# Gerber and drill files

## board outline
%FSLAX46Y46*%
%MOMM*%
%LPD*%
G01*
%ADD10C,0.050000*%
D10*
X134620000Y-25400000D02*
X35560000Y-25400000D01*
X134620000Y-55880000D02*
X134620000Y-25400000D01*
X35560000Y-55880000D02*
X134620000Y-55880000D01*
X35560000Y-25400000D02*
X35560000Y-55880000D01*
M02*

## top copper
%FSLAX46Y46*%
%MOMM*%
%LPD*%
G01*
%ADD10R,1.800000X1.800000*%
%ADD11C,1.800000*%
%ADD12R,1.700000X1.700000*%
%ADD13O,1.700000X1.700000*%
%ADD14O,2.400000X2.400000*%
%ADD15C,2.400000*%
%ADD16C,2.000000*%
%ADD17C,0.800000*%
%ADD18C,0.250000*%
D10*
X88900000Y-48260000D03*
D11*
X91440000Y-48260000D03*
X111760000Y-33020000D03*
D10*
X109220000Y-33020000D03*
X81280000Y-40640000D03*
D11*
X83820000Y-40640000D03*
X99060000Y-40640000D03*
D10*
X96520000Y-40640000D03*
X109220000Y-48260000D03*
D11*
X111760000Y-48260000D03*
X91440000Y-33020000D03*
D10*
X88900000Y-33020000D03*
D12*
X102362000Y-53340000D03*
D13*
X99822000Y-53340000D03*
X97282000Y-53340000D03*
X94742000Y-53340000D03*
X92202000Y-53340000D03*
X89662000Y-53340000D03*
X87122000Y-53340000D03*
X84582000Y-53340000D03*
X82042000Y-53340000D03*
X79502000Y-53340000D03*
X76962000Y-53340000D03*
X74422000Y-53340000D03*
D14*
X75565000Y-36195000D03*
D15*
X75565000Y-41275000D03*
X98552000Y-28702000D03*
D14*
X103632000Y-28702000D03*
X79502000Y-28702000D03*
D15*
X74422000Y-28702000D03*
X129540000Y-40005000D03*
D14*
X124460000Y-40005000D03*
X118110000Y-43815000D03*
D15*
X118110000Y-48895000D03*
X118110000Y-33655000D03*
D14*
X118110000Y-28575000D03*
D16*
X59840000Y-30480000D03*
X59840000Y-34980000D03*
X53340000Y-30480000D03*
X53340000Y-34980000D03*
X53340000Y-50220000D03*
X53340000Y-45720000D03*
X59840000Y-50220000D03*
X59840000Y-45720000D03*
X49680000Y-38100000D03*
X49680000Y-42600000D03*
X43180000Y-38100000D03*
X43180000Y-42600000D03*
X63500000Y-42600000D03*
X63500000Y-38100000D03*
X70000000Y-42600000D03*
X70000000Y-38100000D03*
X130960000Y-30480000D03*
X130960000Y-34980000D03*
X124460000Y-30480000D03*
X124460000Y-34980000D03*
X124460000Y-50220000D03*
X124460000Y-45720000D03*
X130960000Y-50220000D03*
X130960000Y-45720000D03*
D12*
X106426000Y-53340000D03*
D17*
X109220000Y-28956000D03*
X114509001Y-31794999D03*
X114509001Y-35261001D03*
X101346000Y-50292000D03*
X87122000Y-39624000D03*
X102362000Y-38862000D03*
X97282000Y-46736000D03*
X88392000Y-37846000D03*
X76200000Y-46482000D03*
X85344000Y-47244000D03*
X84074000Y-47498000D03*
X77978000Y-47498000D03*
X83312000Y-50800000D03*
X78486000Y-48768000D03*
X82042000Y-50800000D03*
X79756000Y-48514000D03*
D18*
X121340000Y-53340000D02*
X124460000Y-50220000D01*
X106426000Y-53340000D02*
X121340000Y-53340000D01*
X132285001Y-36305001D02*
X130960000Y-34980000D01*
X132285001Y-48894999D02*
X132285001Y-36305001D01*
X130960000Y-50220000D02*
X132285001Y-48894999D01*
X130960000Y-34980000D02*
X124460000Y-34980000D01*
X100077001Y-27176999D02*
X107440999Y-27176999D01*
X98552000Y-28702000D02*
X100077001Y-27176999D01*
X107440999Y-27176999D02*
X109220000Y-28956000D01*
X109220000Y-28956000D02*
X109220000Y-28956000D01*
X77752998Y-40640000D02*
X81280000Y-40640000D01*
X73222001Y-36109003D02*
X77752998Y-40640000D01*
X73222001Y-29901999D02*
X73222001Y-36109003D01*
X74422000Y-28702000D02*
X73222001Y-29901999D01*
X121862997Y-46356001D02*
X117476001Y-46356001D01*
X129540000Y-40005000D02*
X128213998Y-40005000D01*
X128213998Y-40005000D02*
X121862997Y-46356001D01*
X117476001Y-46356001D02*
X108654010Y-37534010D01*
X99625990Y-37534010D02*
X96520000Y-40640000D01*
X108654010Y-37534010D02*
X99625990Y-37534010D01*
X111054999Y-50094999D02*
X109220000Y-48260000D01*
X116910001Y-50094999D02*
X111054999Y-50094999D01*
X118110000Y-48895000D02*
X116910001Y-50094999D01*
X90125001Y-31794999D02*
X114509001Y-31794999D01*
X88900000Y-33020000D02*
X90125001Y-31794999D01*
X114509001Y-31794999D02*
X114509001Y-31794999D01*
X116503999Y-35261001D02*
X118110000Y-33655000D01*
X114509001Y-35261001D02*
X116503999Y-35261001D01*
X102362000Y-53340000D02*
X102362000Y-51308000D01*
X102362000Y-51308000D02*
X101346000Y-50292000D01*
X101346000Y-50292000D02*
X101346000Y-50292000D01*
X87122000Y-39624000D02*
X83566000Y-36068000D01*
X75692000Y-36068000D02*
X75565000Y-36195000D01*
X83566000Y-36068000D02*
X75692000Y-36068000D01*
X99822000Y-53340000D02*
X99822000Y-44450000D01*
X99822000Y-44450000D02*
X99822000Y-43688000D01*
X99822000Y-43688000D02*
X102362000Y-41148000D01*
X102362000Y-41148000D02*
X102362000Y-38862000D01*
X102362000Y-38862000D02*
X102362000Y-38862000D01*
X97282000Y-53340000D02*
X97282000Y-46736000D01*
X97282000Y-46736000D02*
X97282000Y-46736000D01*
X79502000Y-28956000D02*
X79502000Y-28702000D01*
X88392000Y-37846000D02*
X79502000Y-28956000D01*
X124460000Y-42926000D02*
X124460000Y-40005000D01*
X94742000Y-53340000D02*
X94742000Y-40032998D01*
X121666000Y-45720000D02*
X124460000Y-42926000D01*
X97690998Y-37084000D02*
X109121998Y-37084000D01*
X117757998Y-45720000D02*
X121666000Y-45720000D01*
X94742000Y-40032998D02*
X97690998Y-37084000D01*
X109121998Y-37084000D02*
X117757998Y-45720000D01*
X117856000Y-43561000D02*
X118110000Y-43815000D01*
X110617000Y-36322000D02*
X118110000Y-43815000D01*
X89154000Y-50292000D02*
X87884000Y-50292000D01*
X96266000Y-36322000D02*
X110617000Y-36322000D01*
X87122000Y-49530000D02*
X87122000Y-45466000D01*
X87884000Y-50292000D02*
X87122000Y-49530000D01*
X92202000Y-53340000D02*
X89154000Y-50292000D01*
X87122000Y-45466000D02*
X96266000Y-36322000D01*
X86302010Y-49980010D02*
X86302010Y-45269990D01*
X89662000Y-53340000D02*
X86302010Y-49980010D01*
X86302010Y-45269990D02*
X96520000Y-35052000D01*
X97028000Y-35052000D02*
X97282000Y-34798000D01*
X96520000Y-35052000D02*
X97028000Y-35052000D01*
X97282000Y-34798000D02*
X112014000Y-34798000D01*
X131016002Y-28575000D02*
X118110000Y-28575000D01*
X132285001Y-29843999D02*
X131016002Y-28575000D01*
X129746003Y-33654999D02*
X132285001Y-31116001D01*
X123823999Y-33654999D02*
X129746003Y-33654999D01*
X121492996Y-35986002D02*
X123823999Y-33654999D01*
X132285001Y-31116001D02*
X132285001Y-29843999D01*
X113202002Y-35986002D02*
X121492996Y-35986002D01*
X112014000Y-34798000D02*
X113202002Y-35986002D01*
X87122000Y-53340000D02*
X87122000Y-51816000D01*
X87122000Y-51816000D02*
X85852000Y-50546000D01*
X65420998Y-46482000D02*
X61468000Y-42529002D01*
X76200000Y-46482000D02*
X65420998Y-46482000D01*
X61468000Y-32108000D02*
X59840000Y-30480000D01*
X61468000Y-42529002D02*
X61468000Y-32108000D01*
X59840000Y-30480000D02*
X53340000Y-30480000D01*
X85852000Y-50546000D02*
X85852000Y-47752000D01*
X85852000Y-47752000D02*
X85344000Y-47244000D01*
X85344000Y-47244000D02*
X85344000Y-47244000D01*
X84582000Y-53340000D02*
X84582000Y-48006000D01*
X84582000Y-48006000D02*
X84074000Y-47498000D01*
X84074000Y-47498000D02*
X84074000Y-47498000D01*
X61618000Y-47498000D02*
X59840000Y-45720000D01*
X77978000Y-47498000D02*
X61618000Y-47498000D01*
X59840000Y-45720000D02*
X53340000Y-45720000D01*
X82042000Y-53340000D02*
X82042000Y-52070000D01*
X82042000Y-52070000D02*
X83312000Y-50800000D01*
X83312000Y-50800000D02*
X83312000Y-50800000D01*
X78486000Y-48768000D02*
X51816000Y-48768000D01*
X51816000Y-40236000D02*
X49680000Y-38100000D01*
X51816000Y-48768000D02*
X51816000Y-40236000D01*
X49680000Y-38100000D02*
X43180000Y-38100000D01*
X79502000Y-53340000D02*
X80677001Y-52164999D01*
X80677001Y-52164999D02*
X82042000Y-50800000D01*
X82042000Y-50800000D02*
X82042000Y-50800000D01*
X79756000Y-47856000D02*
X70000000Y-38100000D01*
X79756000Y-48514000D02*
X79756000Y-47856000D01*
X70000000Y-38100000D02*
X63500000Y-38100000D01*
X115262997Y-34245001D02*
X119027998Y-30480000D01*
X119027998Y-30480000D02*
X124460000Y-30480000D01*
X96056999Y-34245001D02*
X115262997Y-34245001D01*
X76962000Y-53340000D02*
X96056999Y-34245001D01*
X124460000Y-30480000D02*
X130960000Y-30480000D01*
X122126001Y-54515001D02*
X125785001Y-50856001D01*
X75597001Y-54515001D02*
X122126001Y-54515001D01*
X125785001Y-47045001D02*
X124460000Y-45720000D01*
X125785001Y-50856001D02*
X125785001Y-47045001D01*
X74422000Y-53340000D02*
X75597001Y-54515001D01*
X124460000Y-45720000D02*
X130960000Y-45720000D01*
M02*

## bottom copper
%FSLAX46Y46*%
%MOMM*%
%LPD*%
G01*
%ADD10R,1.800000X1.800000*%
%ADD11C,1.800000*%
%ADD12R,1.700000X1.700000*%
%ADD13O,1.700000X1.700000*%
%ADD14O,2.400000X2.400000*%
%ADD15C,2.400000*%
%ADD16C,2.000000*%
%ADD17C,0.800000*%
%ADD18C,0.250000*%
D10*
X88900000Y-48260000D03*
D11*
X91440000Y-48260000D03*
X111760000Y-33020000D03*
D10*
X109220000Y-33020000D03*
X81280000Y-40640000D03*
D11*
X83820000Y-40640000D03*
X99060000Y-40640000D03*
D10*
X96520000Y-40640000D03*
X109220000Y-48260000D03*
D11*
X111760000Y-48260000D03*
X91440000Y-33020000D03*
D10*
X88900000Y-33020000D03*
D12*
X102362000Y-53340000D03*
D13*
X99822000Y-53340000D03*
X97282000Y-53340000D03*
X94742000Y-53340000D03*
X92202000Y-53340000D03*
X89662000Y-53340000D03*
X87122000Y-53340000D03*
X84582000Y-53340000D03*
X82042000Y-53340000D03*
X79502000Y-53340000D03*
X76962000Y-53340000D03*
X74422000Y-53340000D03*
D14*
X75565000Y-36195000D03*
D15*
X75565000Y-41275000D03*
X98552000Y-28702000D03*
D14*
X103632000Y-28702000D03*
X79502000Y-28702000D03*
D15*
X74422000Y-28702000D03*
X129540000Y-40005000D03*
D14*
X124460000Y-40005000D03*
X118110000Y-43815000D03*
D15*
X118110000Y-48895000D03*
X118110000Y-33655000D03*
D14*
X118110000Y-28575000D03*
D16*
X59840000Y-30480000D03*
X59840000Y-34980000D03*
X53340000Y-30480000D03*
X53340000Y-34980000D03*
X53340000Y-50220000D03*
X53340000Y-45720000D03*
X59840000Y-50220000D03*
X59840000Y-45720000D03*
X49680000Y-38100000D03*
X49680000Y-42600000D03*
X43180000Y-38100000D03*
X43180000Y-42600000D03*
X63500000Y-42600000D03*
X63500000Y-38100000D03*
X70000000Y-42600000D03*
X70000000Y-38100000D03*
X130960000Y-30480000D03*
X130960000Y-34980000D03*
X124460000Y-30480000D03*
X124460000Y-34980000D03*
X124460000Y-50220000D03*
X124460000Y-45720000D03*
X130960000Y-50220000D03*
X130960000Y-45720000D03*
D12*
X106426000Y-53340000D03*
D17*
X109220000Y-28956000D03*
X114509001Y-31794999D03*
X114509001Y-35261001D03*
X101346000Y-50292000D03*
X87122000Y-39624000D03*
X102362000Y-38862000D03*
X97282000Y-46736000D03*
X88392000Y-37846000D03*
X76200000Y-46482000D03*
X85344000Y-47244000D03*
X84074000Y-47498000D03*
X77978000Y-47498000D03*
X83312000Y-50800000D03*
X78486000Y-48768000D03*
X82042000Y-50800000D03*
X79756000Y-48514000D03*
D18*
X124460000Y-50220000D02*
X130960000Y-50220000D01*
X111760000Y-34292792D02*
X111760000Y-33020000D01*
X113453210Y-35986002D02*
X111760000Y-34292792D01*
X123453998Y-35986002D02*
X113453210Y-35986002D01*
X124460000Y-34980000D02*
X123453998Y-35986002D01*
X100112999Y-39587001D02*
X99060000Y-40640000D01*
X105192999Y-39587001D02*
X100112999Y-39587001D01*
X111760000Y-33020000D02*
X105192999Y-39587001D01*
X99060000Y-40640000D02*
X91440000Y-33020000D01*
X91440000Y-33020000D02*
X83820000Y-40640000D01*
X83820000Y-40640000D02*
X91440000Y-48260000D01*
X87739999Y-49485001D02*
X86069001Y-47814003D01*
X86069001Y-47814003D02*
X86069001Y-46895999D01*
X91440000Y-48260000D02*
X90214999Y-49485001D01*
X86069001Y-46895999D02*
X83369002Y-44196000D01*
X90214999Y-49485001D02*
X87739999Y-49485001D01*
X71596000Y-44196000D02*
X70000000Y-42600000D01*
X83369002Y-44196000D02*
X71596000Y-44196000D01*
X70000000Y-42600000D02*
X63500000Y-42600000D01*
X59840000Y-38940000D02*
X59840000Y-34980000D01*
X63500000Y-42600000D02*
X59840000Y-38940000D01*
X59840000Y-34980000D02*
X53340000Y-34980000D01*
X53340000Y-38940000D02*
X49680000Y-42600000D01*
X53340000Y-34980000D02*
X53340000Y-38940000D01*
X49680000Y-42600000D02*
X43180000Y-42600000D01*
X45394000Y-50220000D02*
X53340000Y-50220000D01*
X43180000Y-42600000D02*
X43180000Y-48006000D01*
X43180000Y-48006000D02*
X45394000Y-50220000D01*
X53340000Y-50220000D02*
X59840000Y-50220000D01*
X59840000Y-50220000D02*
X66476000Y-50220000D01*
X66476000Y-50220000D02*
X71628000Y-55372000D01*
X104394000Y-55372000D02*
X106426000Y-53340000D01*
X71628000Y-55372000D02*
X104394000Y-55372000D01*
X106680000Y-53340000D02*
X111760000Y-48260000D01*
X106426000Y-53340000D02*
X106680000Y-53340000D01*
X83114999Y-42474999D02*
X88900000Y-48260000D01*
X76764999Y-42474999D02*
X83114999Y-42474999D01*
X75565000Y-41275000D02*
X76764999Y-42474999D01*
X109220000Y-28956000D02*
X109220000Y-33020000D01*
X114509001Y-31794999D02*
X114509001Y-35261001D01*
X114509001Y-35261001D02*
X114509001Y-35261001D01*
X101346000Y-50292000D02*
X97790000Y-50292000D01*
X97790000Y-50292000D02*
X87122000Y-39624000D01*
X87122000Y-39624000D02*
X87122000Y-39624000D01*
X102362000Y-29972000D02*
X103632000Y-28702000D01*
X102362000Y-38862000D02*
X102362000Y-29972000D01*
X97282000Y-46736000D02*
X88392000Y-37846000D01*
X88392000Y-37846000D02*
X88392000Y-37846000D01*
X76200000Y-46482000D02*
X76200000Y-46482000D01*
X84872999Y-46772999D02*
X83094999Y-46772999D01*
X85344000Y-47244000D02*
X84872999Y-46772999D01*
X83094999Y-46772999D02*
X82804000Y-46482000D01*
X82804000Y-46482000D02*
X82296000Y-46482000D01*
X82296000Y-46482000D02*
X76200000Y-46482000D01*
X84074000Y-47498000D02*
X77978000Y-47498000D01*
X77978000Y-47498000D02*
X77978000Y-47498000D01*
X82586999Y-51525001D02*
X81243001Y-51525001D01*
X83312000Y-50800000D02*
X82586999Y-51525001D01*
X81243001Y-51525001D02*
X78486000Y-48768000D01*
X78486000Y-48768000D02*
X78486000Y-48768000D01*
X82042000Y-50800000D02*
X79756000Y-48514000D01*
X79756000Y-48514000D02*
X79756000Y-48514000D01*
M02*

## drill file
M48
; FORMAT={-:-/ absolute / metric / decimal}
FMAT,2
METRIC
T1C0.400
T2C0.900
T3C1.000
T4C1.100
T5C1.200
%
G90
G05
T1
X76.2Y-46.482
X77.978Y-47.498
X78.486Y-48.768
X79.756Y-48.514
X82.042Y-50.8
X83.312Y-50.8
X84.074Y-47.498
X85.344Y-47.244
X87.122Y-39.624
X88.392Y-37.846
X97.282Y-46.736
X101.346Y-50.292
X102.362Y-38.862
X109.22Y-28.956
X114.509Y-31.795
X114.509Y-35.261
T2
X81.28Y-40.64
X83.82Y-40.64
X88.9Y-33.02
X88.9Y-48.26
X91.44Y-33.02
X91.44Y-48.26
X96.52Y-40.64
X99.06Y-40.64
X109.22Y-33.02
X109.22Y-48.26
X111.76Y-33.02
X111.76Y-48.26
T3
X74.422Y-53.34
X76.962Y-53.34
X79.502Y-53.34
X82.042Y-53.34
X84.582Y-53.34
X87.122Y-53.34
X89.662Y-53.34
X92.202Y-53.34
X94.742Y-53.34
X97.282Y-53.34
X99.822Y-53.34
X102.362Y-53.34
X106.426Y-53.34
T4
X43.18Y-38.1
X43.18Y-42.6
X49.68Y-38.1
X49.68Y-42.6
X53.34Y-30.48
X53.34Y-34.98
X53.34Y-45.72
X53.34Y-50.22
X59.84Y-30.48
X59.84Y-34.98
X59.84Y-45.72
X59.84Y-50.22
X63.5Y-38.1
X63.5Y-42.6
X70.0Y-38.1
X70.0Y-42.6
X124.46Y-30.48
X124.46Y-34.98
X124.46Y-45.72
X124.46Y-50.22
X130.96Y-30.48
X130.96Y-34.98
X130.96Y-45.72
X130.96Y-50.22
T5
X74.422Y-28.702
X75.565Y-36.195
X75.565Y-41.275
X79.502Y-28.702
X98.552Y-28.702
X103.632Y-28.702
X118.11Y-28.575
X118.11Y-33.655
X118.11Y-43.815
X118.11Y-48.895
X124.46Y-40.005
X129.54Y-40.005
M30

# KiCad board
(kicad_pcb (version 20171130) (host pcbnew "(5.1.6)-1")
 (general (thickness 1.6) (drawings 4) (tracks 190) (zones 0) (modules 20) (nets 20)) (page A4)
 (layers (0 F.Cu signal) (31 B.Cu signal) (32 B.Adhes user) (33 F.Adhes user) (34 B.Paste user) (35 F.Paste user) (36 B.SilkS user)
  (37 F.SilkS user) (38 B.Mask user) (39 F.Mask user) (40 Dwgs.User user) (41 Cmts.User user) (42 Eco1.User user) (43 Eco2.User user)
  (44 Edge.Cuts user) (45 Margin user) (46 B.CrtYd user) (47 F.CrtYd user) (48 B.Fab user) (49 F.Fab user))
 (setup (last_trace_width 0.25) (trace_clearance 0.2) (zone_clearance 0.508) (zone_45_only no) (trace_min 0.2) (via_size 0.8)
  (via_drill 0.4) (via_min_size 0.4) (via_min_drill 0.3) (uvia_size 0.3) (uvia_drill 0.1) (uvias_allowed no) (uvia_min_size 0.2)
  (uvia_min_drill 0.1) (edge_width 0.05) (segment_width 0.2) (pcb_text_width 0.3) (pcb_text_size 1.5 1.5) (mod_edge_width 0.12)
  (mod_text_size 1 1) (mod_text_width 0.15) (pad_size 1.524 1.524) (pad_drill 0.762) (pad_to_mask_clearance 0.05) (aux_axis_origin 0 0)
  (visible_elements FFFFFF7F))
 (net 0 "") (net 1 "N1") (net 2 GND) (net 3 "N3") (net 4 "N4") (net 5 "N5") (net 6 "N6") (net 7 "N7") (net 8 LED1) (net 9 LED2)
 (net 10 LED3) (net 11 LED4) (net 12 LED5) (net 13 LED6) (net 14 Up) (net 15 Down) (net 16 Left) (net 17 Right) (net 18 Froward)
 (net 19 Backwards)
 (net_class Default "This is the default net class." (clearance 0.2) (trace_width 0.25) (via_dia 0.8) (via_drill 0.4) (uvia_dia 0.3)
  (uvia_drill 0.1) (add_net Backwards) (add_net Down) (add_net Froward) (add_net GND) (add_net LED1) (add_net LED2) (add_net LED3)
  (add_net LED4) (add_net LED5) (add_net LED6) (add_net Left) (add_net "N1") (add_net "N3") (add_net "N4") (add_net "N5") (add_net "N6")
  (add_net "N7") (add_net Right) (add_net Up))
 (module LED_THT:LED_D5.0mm (layer F.Cu) (at 88.9 48.26)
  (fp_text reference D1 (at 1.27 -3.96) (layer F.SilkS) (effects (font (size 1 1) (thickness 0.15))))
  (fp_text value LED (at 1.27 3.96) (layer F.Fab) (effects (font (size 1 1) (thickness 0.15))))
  (pad 1 thru_hole rect (at 0 0) (size 1.8 1.8) (drill 0.9) (layers *.Cu *.Mask) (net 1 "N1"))
  (pad 2 thru_hole circle (at 2.54 0) (size 1.8 1.8) (drill 0.9) (layers *.Cu *.Mask) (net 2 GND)))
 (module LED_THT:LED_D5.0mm (layer F.Cu) (at 109.22 33.02)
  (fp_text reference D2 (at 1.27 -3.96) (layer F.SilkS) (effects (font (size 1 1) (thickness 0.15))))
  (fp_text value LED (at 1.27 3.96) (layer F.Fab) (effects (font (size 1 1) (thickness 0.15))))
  (pad 2 thru_hole circle (at 2.54 0) (size 1.8 1.8) (drill 0.9) (layers *.Cu *.Mask) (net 2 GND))
  (pad 1 thru_hole rect (at 0 0) (size 1.8 1.8) (drill 0.9) (layers *.Cu *.Mask) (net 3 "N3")))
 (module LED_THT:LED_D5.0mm (layer F.Cu) (at 81.28 40.64)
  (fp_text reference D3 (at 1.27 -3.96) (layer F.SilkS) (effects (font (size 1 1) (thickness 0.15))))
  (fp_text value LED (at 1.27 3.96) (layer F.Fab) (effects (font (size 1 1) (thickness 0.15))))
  (pad 1 thru_hole rect (at 0 0) (size 1.8 1.8) (drill 0.9) (layers *.Cu *.Mask) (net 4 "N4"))
  (pad 2 thru_hole circle (at 2.54 0) (size 1.8 1.8) (drill 0.9) (layers *.Cu *.Mask) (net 2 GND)))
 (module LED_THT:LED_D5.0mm (layer F.Cu) (at 96.52 40.64)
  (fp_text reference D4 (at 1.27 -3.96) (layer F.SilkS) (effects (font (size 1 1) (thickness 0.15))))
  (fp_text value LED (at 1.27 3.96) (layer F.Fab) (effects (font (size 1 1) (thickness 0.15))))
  (pad 2 thru_hole circle (at 2.54 0) (size 1.8 1.8) (drill 0.9) (layers *.Cu *.Mask) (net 2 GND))
  (pad 1 thru_hole rect (at 0 0) (size 1.8 1.8) (drill 0.9) (layers *.Cu *.Mask) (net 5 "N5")))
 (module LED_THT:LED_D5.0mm (layer F.Cu) (at 109.22 48.26)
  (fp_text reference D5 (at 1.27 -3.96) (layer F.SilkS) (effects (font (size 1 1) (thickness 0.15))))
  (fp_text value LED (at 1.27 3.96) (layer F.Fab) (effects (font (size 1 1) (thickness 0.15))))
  (pad 1 thru_hole rect (at 0 0) (size 1.8 1.8) (drill 0.9) (layers *.Cu *.Mask) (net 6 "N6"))
  (pad 2 thru_hole circle (at 2.54 0) (size 1.8 1.8) (drill 0.9) (layers *.Cu *.Mask) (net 2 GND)))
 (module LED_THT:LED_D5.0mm (layer F.Cu) (at 88.9 33.02)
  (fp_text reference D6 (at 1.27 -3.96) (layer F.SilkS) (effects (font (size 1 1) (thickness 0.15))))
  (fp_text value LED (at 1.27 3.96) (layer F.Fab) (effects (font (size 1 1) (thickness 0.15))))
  (pad 2 thru_hole circle (at 2.54 0) (size 1.8 1.8) (drill 0.9) (layers *.Cu *.Mask) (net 2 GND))
  (pad 1 thru_hole rect (at 0 0) (size 1.8 1.8) (drill 0.9) (layers *.Cu *.Mask) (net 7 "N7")))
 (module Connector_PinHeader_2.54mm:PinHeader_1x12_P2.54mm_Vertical (layer F.Cu) (at 102.362 53.34 270)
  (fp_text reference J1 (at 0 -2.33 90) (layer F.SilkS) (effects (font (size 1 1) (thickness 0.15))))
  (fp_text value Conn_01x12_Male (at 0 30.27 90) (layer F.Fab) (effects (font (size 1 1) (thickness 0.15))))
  (pad 1 thru_hole rect (at 0 0 270) (size 1.7 1.7) (drill 1) (layers *.Cu *.Mask) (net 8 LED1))
  (pad 2 thru_hole oval (at 0 2.54 270) (size 1.7 1.7) (drill 1) (layers *.Cu *.Mask) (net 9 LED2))
  (pad 3 thru_hole oval (at 0 5.08 270) (size 1.7 1.7) (drill 1) (layers *.Cu *.Mask) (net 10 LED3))
  (pad 4 thru_hole oval (at 0 7.62 270) (size 1.7 1.7) (drill 1) (layers *.Cu *.Mask) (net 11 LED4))
  (pad 5 thru_hole oval (at 0 10.16 270) (size 1.7 1.7) (drill 1) (layers *.Cu *.Mask) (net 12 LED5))
  (pad 6 thru_hole oval (at 0 12.7 270) (size 1.7 1.7) (drill 1) (layers *.Cu *.Mask) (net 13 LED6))
  (pad 7 thru_hole oval (at 0 15.24 270) (size 1.7 1.7) (drill 1) (layers *.Cu *.Mask) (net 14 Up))
  (pad 8 thru_hole oval (at 0 17.78 270) (size 1.7 1.7) (drill 1) (layers *.Cu *.Mask) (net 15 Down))
  (pad 9 thru_hole oval (at 0 20.32 270) (size 1.7 1.7) (drill 1) (layers *.Cu *.Mask) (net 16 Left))
  (pad 10 thru_hole oval (at 0 22.86 270) (size 1.7 1.7) (drill 1) (layers *.Cu *.Mask) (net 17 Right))
  (pad 11 thru_hole oval (at 0 25.4 270) (size 1.7 1.7) (drill 1) (layers *.Cu *.Mask) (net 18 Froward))
  (pad 12 thru_hole oval (at 0 27.94 270) (size 1.7 1.7) (drill 1) (layers *.Cu *.Mask) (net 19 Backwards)))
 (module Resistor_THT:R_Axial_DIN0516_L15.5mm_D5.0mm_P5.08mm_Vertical (layer F.Cu) (at 75.565 41.275 90)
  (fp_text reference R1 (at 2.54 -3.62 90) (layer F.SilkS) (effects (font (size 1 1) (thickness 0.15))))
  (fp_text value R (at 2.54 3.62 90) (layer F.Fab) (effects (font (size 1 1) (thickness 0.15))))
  (pad 2 thru_hole oval (at 5.08 0 90) (size 2.4 2.4) (drill 1.2) (layers *.Cu *.Mask) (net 8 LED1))
  (pad 1 thru_hole circle (at 0 0 90) (size 2.4 2.4) (drill 1.2) (layers *.Cu *.Mask) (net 1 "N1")))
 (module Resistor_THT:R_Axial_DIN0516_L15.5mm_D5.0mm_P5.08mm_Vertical (layer F.Cu) (at 98.552 28.702)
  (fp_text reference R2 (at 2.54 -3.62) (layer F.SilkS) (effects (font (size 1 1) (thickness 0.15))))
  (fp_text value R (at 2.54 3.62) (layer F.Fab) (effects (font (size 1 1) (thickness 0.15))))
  (pad 1 thru_hole circle (at 0 0) (size 2.4 2.4) (drill 1.2) (layers *.Cu *.Mask) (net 3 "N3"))
  (pad 2 thru_hole oval (at 5.08 0) (size 2.4 2.4) (drill 1.2) (layers *.Cu *.Mask) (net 9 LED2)))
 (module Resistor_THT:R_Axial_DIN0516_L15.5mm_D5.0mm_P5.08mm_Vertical (layer F.Cu) (at 74.422 28.702)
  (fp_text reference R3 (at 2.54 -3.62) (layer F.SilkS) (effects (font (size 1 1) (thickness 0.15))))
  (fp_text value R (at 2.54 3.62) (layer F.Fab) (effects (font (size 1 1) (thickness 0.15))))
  (pad 2 thru_hole oval (at 5.08 0) (size 2.4 2.4) (drill 1.2) (layers *.Cu *.Mask) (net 10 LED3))
  (pad 1 thru_hole circle (at 0 0) (size 2.4 2.4) (drill 1.2) (layers *.Cu *.Mask) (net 4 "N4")))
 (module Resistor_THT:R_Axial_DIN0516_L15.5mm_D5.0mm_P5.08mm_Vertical (layer F.Cu) (at 129.54 40.005 180)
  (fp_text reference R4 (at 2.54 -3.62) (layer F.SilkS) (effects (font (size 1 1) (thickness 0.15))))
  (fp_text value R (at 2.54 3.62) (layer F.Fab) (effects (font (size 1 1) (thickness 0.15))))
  (pad 1 thru_hole circle (at 0 0 180) (size 2.4 2.4) (drill 1.2) (layers *.Cu *.Mask) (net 5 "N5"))
  (pad 2 thru_hole oval (at 5.08 0 180) (size 2.4 2.4) (drill 1.2) (layers *.Cu *.Mask) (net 11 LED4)))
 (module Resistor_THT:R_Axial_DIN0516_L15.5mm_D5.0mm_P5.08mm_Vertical (layer F.Cu) (at 118.11 48.895 90)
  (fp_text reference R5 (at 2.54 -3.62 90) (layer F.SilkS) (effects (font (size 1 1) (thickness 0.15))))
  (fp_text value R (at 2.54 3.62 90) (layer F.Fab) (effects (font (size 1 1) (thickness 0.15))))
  (pad 2 thru_hole oval (at 5.08 0 90) (size 2.4 2.4) (drill 1.2) (layers *.Cu *.Mask) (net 12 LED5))
  (pad 1 thru_hole circle (at 0 0 90) (size 2.4 2.4) (drill 1.2) (layers *.Cu *.Mask) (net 6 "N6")))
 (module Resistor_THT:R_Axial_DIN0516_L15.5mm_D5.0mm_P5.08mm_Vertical (layer F.Cu) (at 118.11 33.655 90)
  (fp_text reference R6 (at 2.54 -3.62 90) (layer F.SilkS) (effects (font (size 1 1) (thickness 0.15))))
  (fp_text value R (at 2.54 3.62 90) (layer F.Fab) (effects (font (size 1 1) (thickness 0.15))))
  (pad 1 thru_hole circle (at 0 0 90) (size 2.4 2.4) (drill 1.2) (layers *.Cu *.Mask) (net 7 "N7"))
  (pad 2 thru_hole oval (at 5.08 0 90) (size 2.4 2.4) (drill 1.2) (layers *.Cu *.Mask) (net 13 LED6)))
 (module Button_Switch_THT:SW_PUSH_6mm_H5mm (layer F.Cu) (at 53.34 30.48)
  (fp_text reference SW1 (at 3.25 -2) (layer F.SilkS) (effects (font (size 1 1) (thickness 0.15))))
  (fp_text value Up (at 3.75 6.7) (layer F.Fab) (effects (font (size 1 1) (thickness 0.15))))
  (pad 1 thru_hole circle (at 6.5 0 90) (size 2 2) (drill 1.1) (layers *.Cu *.Mask) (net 14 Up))
  (pad 2 thru_hole circle (at 6.5 4.5 90) (size 2 2) (drill 1.1) (layers *.Cu *.Mask) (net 2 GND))
  (pad 1 thru_hole circle (at 0 0 90) (size 2 2) (drill 1.1) (layers *.Cu *.Mask) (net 14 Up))
  (pad 2 thru_hole circle (at 0 4.5 90) (size 2 2) (drill 1.1) (layers *.Cu *.Mask) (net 2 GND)))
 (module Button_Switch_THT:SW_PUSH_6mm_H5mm (layer F.Cu) (at 53.34 45.72)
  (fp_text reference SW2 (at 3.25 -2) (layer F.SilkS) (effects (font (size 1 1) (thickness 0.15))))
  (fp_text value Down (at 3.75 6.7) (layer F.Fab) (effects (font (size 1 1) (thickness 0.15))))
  (pad 2 thru_hole circle (at 0 4.5 90) (size 2 2) (drill 1.1) (layers *.Cu *.Mask) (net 2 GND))
  (pad 1 thru_hole circle (at 0 0 90) (size 2 2) (drill 1.1) (layers *.Cu *.Mask) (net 15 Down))
  (pad 2 thru_hole circle (at 6.5 4.5 90) (size 2 2) (drill 1.1) (layers *.Cu *.Mask) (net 2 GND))
  (pad 1 thru_hole circle (at 6.5 0 90) (size 2 2) (drill 1.1) (layers *.Cu *.Mask) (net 15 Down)))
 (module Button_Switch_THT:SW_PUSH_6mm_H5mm (layer F.Cu) (at 43.18 38.1)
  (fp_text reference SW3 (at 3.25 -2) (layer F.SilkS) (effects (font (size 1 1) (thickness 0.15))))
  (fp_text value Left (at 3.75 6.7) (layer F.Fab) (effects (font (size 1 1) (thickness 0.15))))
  (pad 1 thru_hole circle (at 6.5 0 90) (size 2 2) (drill 1.1) (layers *.Cu *.Mask) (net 16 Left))
  (pad 2 thru_hole circle (at 6.5 4.5 90) (size 2 2) (drill 1.1) (layers *.Cu *.Mask) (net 2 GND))
  (pad 1 thru_hole circle (at 0 0 90) (size 2 2) (drill 1.1) (layers *.Cu *.Mask) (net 16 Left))
  (pad 2 thru_hole circle (at 0 4.5 90) (size 2 2) (drill 1.1) (layers *.Cu *.Mask) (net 2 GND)))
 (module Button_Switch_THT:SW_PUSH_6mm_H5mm (layer F.Cu) (at 63.5 38.1)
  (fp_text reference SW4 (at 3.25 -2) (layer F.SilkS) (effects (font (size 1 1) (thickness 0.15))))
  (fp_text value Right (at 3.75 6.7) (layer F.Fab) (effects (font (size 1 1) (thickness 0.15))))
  (pad 2 thru_hole circle (at 0 4.5 90) (size 2 2) (drill 1.1) (layers *.Cu *.Mask) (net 2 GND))
  (pad 1 thru_hole circle (at 0 0 90) (size 2 2) (drill 1.1) (layers *.Cu *.Mask) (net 17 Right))
  (pad 2 thru_hole circle (at 6.5 4.5 90) (size 2 2) (drill 1.1) (layers *.Cu *.Mask) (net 2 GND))
  (pad 1 thru_hole circle (at 6.5 0 90) (size 2 2) (drill 1.1) (layers *.Cu *.Mask) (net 17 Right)))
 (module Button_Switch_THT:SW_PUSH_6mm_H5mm (layer F.Cu) (at 124.46 30.48)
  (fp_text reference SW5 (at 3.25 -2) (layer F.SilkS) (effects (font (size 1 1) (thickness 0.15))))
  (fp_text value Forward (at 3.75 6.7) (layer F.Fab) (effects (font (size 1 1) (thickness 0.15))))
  (pad 1 thru_hole circle (at 6.5 0 90) (size 2 2) (drill 1.1) (layers *.Cu *.Mask) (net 18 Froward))
  (pad 2 thru_hole circle (at 6.5 4.5 90) (size 2 2) (drill 1.1) (layers *.Cu *.Mask) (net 2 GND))
  (pad 1 thru_hole circle (at 0 0 90) (size 2 2) (drill 1.1) (layers *.Cu *.Mask) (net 18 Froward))
  (pad 2 thru_hole circle (at 0 4.5 90) (size 2 2) (drill 1.1) (layers *.Cu *.Mask) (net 2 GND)))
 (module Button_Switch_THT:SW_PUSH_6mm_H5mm (layer F.Cu) (at 124.46 45.72)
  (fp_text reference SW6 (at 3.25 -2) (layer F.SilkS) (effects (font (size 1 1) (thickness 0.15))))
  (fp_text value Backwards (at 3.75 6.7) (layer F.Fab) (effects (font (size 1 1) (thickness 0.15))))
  (pad 2 thru_hole circle (at 0 4.5 90) (size 2 2) (drill 1.1) (layers *.Cu *.Mask) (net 2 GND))
  (pad 1 thru_hole circle (at 0 0 90) (size 2 2) (drill 1.1) (layers *.Cu *.Mask) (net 19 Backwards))
  (pad 2 thru_hole circle (at 6.5 4.5 90) (size 2 2) (drill 1.1) (layers *.Cu *.Mask) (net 2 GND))
  (pad 1 thru_hole circle (at 6.5 0 90) (size 2 2) (drill 1.1) (layers *.Cu *.Mask) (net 19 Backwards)))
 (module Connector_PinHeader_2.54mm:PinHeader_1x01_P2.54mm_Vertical (layer F.Cu) (at 106.426 53.34)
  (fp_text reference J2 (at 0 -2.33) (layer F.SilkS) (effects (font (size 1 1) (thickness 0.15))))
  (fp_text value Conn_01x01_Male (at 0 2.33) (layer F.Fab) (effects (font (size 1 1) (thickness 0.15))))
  (pad 1 thru_hole rect (at 0 0) (size 1.7 1.7) (drill 1) (layers *.Cu *.Mask) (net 2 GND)))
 (gr_line (start 134.62 25.4) (end 35.56 25.4) (layer Edge.Cuts) (width 0.05))
 (gr_line (start 134.62 55.88) (end 134.62 25.4) (layer Edge.Cuts) (width 0.05))
 (gr_line (start 35.56 55.88) (end 134.62 55.88) (layer Edge.Cuts) (width 0.05))
 (gr_line (start 35.56 25.4) (end 35.56 55.88) (layer Edge.Cuts) (width 0.05))
 (segment (start 121.34 53.34) (end 124.46 50.22) (width 0.25) (layer F.Cu) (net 2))
 (segment (start 106.426 53.34) (end 121.34 53.34) (width 0.25) (layer F.Cu) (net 2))
 (segment (start 124.46 50.22) (end 130.96 50.22) (width 0.25) (layer B.Cu) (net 2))
 (segment (start 132.285001 36.305001) (end 130.96 34.98) (width 0.25) (layer F.Cu) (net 2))
 (segment (start 132.285001 48.894999) (end 132.285001 36.305001) (width 0.25) (layer F.Cu) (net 2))
 (segment (start 130.96 50.22) (end 132.285001 48.894999) (width 0.25) (layer F.Cu) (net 2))
 (segment (start 130.96 34.98) (end 124.46 34.98) (width 0.25) (layer F.Cu) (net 2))
 (segment (start 111.76 34.292792) (end 111.76 33.02) (width 0.25) (layer B.Cu) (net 2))
 (segment (start 113.45321 35.986002) (end 111.76 34.292792) (width 0.25) (layer B.Cu) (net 2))
 (segment (start 123.453998 35.986002) (end 113.45321 35.986002) (width 0.25) (layer B.Cu) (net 2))
 (segment (start 124.46 34.98) (end 123.453998 35.986002) (width 0.25) (layer B.Cu) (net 2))
 (segment (start 100.112999 39.587001) (end 99.06 40.64) (width 0.25) (layer B.Cu) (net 2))
 (segment (start 105.192999 39.587001) (end 100.112999 39.587001) (width 0.25) (layer B.Cu) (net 2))
 (segment (start 111.76 33.02) (end 105.192999 39.587001) (width 0.25) (layer B.Cu) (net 2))
 (segment (start 99.06 40.64) (end 91.44 33.02) (width 0.25) (layer B.Cu) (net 2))
 (segment (start 91.44 33.02) (end 83.82 40.64) (width 0.25) (layer B.Cu) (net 2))
 (segment (start 83.82 40.64) (end 91.44 48.26) (width 0.25) (layer B.Cu) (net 2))
 (segment (start 87.739999 49.485001) (end 86.069001 47.814003) (width 0.25) (layer B.Cu) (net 2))
 (segment (start 86.069001 47.814003) (end 86.069001 46.895999) (width 0.25) (layer B.Cu) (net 2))
 (segment (start 91.44 48.26) (end 90.214999 49.485001) (width 0.25) (layer B.Cu) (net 2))
 (segment (start 86.069001 46.895999) (end 83.369002 44.196) (width 0.25) (layer B.Cu) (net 2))
 (segment (start 90.214999 49.485001) (end 87.739999 49.485001) (width 0.25) (layer B.Cu) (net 2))
 (segment (start 71.596 44.196) (end 70 42.6) (width 0.25) (layer B.Cu) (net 2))
 (segment (start 83.369002 44.196) (end 71.596 44.196) (width 0.25) (layer B.Cu) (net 2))
 (segment (start 70 42.6) (end 63.5 42.6) (width 0.25) (layer B.Cu) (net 2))
 (segment (start 59.84 38.94) (end 59.84 34.98) (width 0.25) (layer B.Cu) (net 2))
 (segment (start 63.5 42.6) (end 59.84 38.94) (width 0.25) (layer B.Cu) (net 2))
 (segment (start 59.84 34.98) (end 53.34 34.98) (width 0.25) (layer B.Cu) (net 2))
 (segment (start 53.34 38.94) (end 49.68 42.6) (width 0.25) (layer B.Cu) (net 2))
 (segment (start 53.34 34.98) (end 53.34 38.94) (width 0.25) (layer B.Cu) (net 2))
 (segment (start 49.68 42.6) (end 43.18 42.6) (width 0.25) (layer B.Cu) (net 2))
 (segment (start 45.394 50.22) (end 53.34 50.22) (width 0.25) (layer B.Cu) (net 2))
 (segment (start 43.18 42.6) (end 43.18 48.006) (width 0.25) (layer B.Cu) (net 2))
 (segment (start 43.18 48.006) (end 45.394 50.22) (width 0.25) (layer B.Cu) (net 2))
 (segment (start 53.34 50.22) (end 59.84 50.22) (width 0.25) (layer B.Cu) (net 2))
 (segment (start 59.84 50.22) (end 66.476 50.22) (width 0.25) (layer B.Cu) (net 2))
 (segment (start 66.476 50.22) (end 71.628 55.372) (width 0.25) (layer B.Cu) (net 2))
 (segment (start 104.394 55.372) (end 106.426 53.34) (width 0.25) (layer B.Cu) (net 2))
 (segment (start 71.628 55.372) (end 104.394 55.372) (width 0.25) (layer B.Cu) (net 2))
 (segment (start 106.68 53.34) (end 111.76 48.26) (width 0.25) (layer B.Cu) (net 2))
 (segment (start 106.426 53.34) (end 106.68 53.34) (width 0.25) (layer B.Cu) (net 2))
 (segment (start 83.114999 42.474999) (end 88.9 48.26) (width 0.25) (layer B.Cu) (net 1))
 (segment (start 76.764999 42.474999) (end 83.114999 42.474999) (width 0.25) (layer B.Cu) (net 1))
 (segment (start 75.565 41.275) (end 76.764999 42.474999) (width 0.25) (layer B.Cu) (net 1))
 (segment (start 100.077001 27.176999) (end 107.440999 27.176999) (width 0.25) (layer F.Cu) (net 3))
 (segment (start 98.552 28.702) (end 100.077001 27.176999) (width 0.25) (layer F.Cu) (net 3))
 (segment (start 107.440999 27.176999) (end 109.22 28.956) (width 0.25) (layer F.Cu) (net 3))
 (segment (start 109.22 28.956) (end 109.22 28.956) (width 0.25) (layer F.Cu) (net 3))
 (via (at 109.22 28.956) (size 0.8) (drill 0.4) (layers F.Cu B.Cu) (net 3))
 (segment (start 109.22 28.956) (end 109.22 33.02) (width 0.25) (layer B.Cu) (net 3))
 (segment (start 77.752998 40.64) (end 81.28 40.64) (width 0.25) (layer F.Cu) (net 4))
 (segment (start 73.222001 36.109003) (end 77.752998 40.64) (width 0.25) (layer F.Cu) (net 4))
 (segment (start 73.222001 29.901999) (end 73.222001 36.109003) (width 0.25) (layer F.Cu) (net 4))
 (segment (start 74.422 28.702) (end 73.222001 29.901999) (width 0.25) (layer F.Cu) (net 4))
 (segment (start 121.862997 46.356001) (end 117.476001 46.356001) (width 0.25) (layer F.Cu) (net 5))
 (segment (start 129.54 40.005) (end 128.213998 40.005) (width 0.25) (layer F.Cu) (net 5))
 (segment (start 128.213998 40.005) (end 121.862997 46.356001) (width 0.25) (layer F.Cu) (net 5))
 (segment (start 117.476001 46.356001) (end 108.65401 37.53401) (width 0.25) (layer F.Cu) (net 5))
 (segment (start 99.62599 37.53401) (end 96.52 40.64) (width 0.25) (layer F.Cu) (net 5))
 (segment (start 108.65401 37.53401) (end 99.62599 37.53401) (width 0.25) (layer F.Cu) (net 5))
 (segment (start 111.054999 50.094999) (end 109.22 48.26) (width 0.25) (layer F.Cu) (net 6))
 (segment (start 116.910001 50.094999) (end 111.054999 50.094999) (width 0.25) (layer F.Cu) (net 6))
 (segment (start 118.11 48.895) (end 116.910001 50.094999) (width 0.25) (layer F.Cu) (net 6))
 (segment (start 90.125001 31.794999) (end 114.509001 31.794999) (width 0.25) (layer F.Cu) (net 7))
 (segment (start 88.9 33.02) (end 90.125001 31.794999) (width 0.25) (layer F.Cu) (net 7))
 (segment (start 114.509001 31.794999) (end 114.509001 31.794999) (width 0.25) (layer F.Cu) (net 7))
 (via (at 114.509001 31.794999) (size 0.8) (drill 0.4) (layers F.Cu B.Cu) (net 7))
 (segment (start 114.509001 31.794999) (end 114.509001 35.261001) (width 0.25) (layer B.Cu) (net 7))
 (segment (start 114.509001 35.261001) (end 114.509001 35.261001) (width 0.25) (layer B.Cu) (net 7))
 (via (at 114.509001 35.261001) (size 0.8) (drill 0.4) (layers F.Cu B.Cu) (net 7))
 (segment (start 116.503999 35.261001) (end 118.11 33.655) (width 0.25) (layer F.Cu) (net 7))
 (segment (start 114.509001 35.261001) (end 116.503999 35.261001) (width 0.25) (layer F.Cu) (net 7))
 (segment (start 102.362 53.34) (end 102.362 51.308) (width 0.25) (layer F.Cu) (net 8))
 (segment (start 102.362 51.308) (end 101.346 50.292) (width 0.25) (layer F.Cu) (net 8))
 (segment (start 101.346 50.292) (end 101.346 50.292) (width 0.25) (layer F.Cu) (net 8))
 (via (at 101.346 50.292) (size 0.8) (drill 0.4) (layers F.Cu B.Cu) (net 8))
 (segment (start 101.346 50.292) (end 97.79 50.292) (width 0.25) (layer B.Cu) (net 8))
 (segment (start 97.79 50.292) (end 87.122 39.624) (width 0.25) (layer B.Cu) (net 8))
 (segment (start 87.122 39.624) (end 87.122 39.624) (width 0.25) (layer B.Cu) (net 8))
 (via (at 87.122 39.624) (size 0.8) (drill 0.4) (layers F.Cu B.Cu) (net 8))
 (segment (start 87.122 39.624) (end 83.566 36.068) (width 0.25) (layer F.Cu) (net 8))
 (segment (start 75.692 36.068) (end 75.565 36.195) (width 0.25) (layer F.Cu) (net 8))
 (segment (start 83.566 36.068) (end 75.692 36.068) (width 0.25) (layer F.Cu) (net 8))
 (segment (start 99.822 53.34) (end 99.822 44.45) (width 0.25) (layer F.Cu) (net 9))
 (segment (start 99.822 44.45) (end 99.822 43.688) (width 0.25) (layer F.Cu) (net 9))
 (segment (start 99.822 43.688) (end 102.362 41.148) (width 0.25) (layer F.Cu) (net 9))
 (segment (start 102.362 41.148) (end 102.362 38.862) (width 0.25) (layer F.Cu) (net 9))
 (segment (start 102.362 38.862) (end 102.362 38.862) (width 0.25) (layer F.Cu) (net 9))
 (via (at 102.362 38.862) (size 0.8) (drill 0.4) (layers F.Cu B.Cu) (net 9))
 (segment (start 102.362 29.972) (end 103.632 28.702) (width 0.25) (layer B.Cu) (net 9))
 (segment (start 102.362 38.862) (end 102.362 29.972) (width 0.25) (layer B.Cu) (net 9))
 (segment (start 97.282 53.34) (end 97.282 46.736) (width 0.25) (layer F.Cu) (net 10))
 (segment (start 97.282 46.736) (end 97.282 46.736) (width 0.25) (layer F.Cu) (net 10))
 (via (at 97.282 46.736) (size 0.8) (drill 0.4) (layers F.Cu B.Cu) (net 10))
 (segment (start 97.282 46.736) (end 88.392 37.846) (width 0.25) (layer B.Cu) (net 10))
 (segment (start 88.392 37.846) (end 88.392 37.846) (width 0.25) (layer B.Cu) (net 10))
 (via (at 88.392 37.846) (size 0.8) (drill 0.4) (layers F.Cu B.Cu) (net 10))
 (segment (start 79.502 28.956) (end 79.502 28.702) (width 0.25) (layer F.Cu) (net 10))
 (segment (start 88.392 37.846) (end 79.502 28.956) (width 0.25) (layer F.Cu) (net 10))
 (segment (start 124.46 42.926) (end 124.46 40.005) (width 0.25) (layer F.Cu) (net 11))
 (segment (start 94.742 53.34) (end 94.742 40.032998) (width 0.25) (layer F.Cu) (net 11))
 (segment (start 121.666 45.72) (end 124.46 42.926) (width 0.25) (layer F.Cu) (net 11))
 (segment (start 97.690998 37.084) (end 109.121998 37.084) (width 0.25) (layer F.Cu) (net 11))
 (segment (start 117.757998 45.72) (end 121.666 45.72) (width 0.25) (layer F.Cu) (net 11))
 (segment (start 94.742 40.032998) (end 97.690998 37.084) (width 0.25) (layer F.Cu) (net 11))
 (segment (start 109.121998 37.084) (end 117.757998 45.72) (width 0.25) (layer F.Cu) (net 11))
 (segment (start 117.856 43.561) (end 118.11 43.815) (width 0.25) (layer F.Cu) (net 12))
 (segment (start 110.617 36.322) (end 118.11 43.815) (width 0.25) (layer F.Cu) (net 12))
 (segment (start 89.154 50.292) (end 87.884 50.292) (width 0.25) (layer F.Cu) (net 12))
 (segment (start 96.266 36.322) (end 110.617 36.322) (width 0.25) (layer F.Cu) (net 12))
 (segment (start 87.122 49.53) (end 87.122 45.466) (width 0.25) (layer F.Cu) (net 12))
 (segment (start 87.884 50.292) (end 87.122 49.53) (width 0.25) (layer F.Cu) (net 12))
 (segment (start 92.202 53.34) (end 89.154 50.292) (width 0.25) (layer F.Cu) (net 12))
 (segment (start 87.122 45.466) (end 96.266 36.322) (width 0.25) (layer F.Cu) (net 12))
 (segment (start 86.30201 49.98001) (end 86.30201 45.26999) (width 0.25) (layer F.Cu) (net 13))
 (segment (start 89.662 53.34) (end 86.30201 49.98001) (width 0.25) (layer F.Cu) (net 13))
 (segment (start 86.30201 45.26999) (end 96.52 35.052) (width 0.25) (layer F.Cu) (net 13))
 (segment (start 97.028 35.052) (end 97.282 34.798) (width 0.25) (layer F.Cu) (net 13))
 (segment (start 96.52 35.052) (end 97.028 35.052) (width 0.25) (layer F.Cu) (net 13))
 (segment (start 97.282 34.798) (end 112.014 34.798) (width 0.25) (layer F.Cu) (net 13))
 (segment (start 131.016002 28.575) (end 118.11 28.575) (width 0.25) (layer F.Cu) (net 13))
 (segment (start 132.285001 29.843999) (end 131.016002 28.575) (width 0.25) (layer F.Cu) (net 13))
 (segment (start 129.746003 33.654999) (end 132.285001 31.116001) (width 0.25) (layer F.Cu) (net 13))
 (segment (start 123.823999 33.654999) (end 129.746003 33.654999) (width 0.25) (layer F.Cu) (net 13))
 (segment (start 121.492996 35.986002) (end 123.823999 33.654999) (width 0.25) (layer F.Cu) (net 13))
 (segment (start 132.285001 31.116001) (end 132.285001 29.843999) (width 0.25) (layer F.Cu) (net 13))
 (segment (start 113.202002 35.986002) (end 121.492996 35.986002) (width 0.25) (layer F.Cu) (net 13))
 (segment (start 112.014 34.798) (end 113.202002 35.986002) (width 0.25) (layer F.Cu) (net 13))
 (segment (start 87.122 53.34) (end 87.122 51.816) (width 0.25) (layer F.Cu) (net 14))
 (segment (start 87.122 51.816) (end 85.852 50.546) (width 0.25) (layer F.Cu) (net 14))
 (segment (start 76.2 46.482) (end 76.2 46.482) (width 0.25) (layer B.Cu) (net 14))
 (via (at 76.2 46.482) (size 0.8) (drill 0.4) (layers F.Cu B.Cu) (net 14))
 (segment (start 65.420998 46.482) (end 61.468 42.529002) (width 0.25) (layer F.Cu) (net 14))
 (segment (start 76.2 46.482) (end 65.420998 46.482) (width 0.25) (layer F.Cu) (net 14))
 (segment (start 61.468 32.108) (end 59.84 30.48) (width 0.25) (layer F.Cu) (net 14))
 (segment (start 61.468 42.529002) (end 61.468 32.108) (width 0.25) (layer F.Cu) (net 14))
 (segment (start 59.84 30.48) (end 53.34 30.48) (width 0.25) (layer F.Cu) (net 14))
 (segment (start 85.852 50.546) (end 85.852 47.752) (width 0.25) (layer F.Cu) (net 14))
 (segment (start 85.852 47.752) (end 85.344 47.244) (width 0.25) (layer F.Cu) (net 14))
 (segment (start 85.344 47.244) (end 85.344 47.244) (width 0.25) (layer F.Cu) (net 14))
 (via (at 85.344 47.244) (size 0.8) (drill 0.4) (layers F.Cu B.Cu) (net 14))
 (segment (start 84.872999 46.772999) (end 83.094999 46.772999) (width 0.25) (layer B.Cu) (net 14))
 (segment (start 85.344 47.244) (end 84.872999 46.772999) (width 0.25) (layer B.Cu) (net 14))
 (segment (start 83.094999 46.772999) (end 82.804 46.482) (width 0.25) (layer B.Cu) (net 14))
 (segment (start 82.804 46.482) (end 82.296 46.482) (width 0.25) (layer B.Cu) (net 14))
 (segment (start 82.296 46.482) (end 76.2 46.482) (width 0.25) (layer B.Cu) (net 14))
 (segment (start 84.582 53.34) (end 84.582 48.006) (width 0.25) (layer F.Cu) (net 15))
 (segment (start 84.582 48.006) (end 84.074 47.498) (width 0.25) (layer F.Cu) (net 15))
 (segment (start 84.074 47.498) (end 84.074 47.498) (width 0.25) (layer F.Cu) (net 15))
 (via (at 84.074 47.498) (size 0.8) (drill 0.4) (layers F.Cu B.Cu) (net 15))
 (segment (start 84.074 47.498) (end 77.978 47.498) (width 0.25) (layer B.Cu) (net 15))
 (segment (start 77.978 47.498) (end 77.978 47.498) (width 0.25) (layer B.Cu) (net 15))
 (via (at 77.978 47.498) (size 0.8) (drill 0.4) (layers F.Cu B.Cu) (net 15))
 (segment (start 61.618 47.498) (end 59.84 45.72) (width 0.25) (layer F.Cu) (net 15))
 (segment (start 77.978 47.498) (end 61.618 47.498) (width 0.25) (layer F.Cu) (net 15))
 (segment (start 59.84 45.72) (end 53.34 45.72) (width 0.25) (layer F.Cu) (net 15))
 (segment (start 82.042 53.34) (end 82.042 52.07) (width 0.25) (layer F.Cu) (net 16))
 (segment (start 82.042 52.07) (end 83.312 50.8) (width 0.25) (layer F.Cu) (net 16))
 (segment (start 83.312 50.8) (end 83.312 50.8) (width 0.25) (layer F.Cu) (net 16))
 (via (at 83.312 50.8) (size 0.8) (drill 0.4) (layers F.Cu B.Cu) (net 16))
 (segment (start 82.586999 51.525001) (end 81.243001 51.525001) (width 0.25) (layer B.Cu) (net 16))
 (segment (start 83.312 50.8) (end 82.586999 51.525001) (width 0.25) (layer B.Cu) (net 16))
 (segment (start 81.243001 51.525001) (end 78.486 48.768) (width 0.25) (layer B.Cu) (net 16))
 (segment (start 78.486 48.768) (end 78.486 48.768) (width 0.25) (layer B.Cu) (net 16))
 (via (at 78.486 48.768) (size 0.8) (drill 0.4) (layers F.Cu B.Cu) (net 16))
 (segment (start 78.486 48.768) (end 51.816 48.768) (width 0.25) (layer F.Cu) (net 16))
 (segment (start 51.816 40.236) (end 49.68 38.1) (width 0.25) (layer F.Cu) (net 16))
 (segment (start 51.816 48.768) (end 51.816 40.236) (width 0.25) (layer F.Cu) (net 16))
 (segment (start 49.68 38.1) (end 43.18 38.1) (width 0.25) (layer F.Cu) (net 16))
 (segment (start 79.502 53.34) (end 80.677001 52.164999) (width 0.25) (layer F.Cu) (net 17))
 (segment (start 80.677001 52.164999) (end 82.042 50.8) (width 0.25) (layer F.Cu) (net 17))
 (segment (start 82.042 50.8) (end 82.042 50.8) (width 0.25) (layer F.Cu) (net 17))
 (via (at 82.042 50.8) (size 0.8) (drill 0.4) (layers F.Cu B.Cu) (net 17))
 (segment (start 82.042 50.8) (end 79.756 48.514) (width 0.25) (layer B.Cu) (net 17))
 (segment (start 79.756 48.514) (end 79.756 48.514) (width 0.25) (layer B.Cu) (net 17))
 (via (at 79.756 48.514) (size 0.8) (drill 0.4) (layers F.Cu B.Cu) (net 17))
 (segment (start 79.756 47.856) (end 70 38.1) (width 0.25) (layer F.Cu) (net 17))
 (segment (start 79.756 48.514) (end 79.756 47.856) (width 0.25) (layer F.Cu) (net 17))
 (segment (start 70 38.1) (end 63.5 38.1) (width 0.25) (layer F.Cu) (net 17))
 (segment (start 115.262997 34.245001) (end 119.027998 30.48) (width 0.25) (layer F.Cu) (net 18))
 (segment (start 119.027998 30.48) (end 124.46 30.48) (width 0.25) (layer F.Cu) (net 18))
 (segment (start 96.056999 34.245001) (end 115.262997 34.245001) (width 0.25) (layer F.Cu) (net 18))
 (segment (start 76.962 53.34) (end 96.056999 34.245001) (width 0.25) (layer F.Cu) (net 18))
 (segment (start 124.46 30.48) (end 130.96 30.48) (width 0.25) (layer F.Cu) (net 18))
 (segment (start 122.126001 54.515001) (end 125.785001 50.856001) (width 0.25) (layer F.Cu) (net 19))
 (segment (start 75.597001 54.515001) (end 122.126001 54.515001) (width 0.25) (layer F.Cu) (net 19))
 (segment (start 125.785001 47.045001) (end 124.46 45.72) (width 0.25) (layer F.Cu) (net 19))
 (segment (start 125.785001 50.856001) (end 125.785001 47.045001) (width 0.25) (layer F.Cu) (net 19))
 (segment (start 74.422 53.34) (end 75.597001 54.515001) (width 0.25) (layer F.Cu) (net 19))
 (segment (start 124.46 45.72) (end 130.96 45.72) (width 0.25) (layer F.Cu) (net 19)))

